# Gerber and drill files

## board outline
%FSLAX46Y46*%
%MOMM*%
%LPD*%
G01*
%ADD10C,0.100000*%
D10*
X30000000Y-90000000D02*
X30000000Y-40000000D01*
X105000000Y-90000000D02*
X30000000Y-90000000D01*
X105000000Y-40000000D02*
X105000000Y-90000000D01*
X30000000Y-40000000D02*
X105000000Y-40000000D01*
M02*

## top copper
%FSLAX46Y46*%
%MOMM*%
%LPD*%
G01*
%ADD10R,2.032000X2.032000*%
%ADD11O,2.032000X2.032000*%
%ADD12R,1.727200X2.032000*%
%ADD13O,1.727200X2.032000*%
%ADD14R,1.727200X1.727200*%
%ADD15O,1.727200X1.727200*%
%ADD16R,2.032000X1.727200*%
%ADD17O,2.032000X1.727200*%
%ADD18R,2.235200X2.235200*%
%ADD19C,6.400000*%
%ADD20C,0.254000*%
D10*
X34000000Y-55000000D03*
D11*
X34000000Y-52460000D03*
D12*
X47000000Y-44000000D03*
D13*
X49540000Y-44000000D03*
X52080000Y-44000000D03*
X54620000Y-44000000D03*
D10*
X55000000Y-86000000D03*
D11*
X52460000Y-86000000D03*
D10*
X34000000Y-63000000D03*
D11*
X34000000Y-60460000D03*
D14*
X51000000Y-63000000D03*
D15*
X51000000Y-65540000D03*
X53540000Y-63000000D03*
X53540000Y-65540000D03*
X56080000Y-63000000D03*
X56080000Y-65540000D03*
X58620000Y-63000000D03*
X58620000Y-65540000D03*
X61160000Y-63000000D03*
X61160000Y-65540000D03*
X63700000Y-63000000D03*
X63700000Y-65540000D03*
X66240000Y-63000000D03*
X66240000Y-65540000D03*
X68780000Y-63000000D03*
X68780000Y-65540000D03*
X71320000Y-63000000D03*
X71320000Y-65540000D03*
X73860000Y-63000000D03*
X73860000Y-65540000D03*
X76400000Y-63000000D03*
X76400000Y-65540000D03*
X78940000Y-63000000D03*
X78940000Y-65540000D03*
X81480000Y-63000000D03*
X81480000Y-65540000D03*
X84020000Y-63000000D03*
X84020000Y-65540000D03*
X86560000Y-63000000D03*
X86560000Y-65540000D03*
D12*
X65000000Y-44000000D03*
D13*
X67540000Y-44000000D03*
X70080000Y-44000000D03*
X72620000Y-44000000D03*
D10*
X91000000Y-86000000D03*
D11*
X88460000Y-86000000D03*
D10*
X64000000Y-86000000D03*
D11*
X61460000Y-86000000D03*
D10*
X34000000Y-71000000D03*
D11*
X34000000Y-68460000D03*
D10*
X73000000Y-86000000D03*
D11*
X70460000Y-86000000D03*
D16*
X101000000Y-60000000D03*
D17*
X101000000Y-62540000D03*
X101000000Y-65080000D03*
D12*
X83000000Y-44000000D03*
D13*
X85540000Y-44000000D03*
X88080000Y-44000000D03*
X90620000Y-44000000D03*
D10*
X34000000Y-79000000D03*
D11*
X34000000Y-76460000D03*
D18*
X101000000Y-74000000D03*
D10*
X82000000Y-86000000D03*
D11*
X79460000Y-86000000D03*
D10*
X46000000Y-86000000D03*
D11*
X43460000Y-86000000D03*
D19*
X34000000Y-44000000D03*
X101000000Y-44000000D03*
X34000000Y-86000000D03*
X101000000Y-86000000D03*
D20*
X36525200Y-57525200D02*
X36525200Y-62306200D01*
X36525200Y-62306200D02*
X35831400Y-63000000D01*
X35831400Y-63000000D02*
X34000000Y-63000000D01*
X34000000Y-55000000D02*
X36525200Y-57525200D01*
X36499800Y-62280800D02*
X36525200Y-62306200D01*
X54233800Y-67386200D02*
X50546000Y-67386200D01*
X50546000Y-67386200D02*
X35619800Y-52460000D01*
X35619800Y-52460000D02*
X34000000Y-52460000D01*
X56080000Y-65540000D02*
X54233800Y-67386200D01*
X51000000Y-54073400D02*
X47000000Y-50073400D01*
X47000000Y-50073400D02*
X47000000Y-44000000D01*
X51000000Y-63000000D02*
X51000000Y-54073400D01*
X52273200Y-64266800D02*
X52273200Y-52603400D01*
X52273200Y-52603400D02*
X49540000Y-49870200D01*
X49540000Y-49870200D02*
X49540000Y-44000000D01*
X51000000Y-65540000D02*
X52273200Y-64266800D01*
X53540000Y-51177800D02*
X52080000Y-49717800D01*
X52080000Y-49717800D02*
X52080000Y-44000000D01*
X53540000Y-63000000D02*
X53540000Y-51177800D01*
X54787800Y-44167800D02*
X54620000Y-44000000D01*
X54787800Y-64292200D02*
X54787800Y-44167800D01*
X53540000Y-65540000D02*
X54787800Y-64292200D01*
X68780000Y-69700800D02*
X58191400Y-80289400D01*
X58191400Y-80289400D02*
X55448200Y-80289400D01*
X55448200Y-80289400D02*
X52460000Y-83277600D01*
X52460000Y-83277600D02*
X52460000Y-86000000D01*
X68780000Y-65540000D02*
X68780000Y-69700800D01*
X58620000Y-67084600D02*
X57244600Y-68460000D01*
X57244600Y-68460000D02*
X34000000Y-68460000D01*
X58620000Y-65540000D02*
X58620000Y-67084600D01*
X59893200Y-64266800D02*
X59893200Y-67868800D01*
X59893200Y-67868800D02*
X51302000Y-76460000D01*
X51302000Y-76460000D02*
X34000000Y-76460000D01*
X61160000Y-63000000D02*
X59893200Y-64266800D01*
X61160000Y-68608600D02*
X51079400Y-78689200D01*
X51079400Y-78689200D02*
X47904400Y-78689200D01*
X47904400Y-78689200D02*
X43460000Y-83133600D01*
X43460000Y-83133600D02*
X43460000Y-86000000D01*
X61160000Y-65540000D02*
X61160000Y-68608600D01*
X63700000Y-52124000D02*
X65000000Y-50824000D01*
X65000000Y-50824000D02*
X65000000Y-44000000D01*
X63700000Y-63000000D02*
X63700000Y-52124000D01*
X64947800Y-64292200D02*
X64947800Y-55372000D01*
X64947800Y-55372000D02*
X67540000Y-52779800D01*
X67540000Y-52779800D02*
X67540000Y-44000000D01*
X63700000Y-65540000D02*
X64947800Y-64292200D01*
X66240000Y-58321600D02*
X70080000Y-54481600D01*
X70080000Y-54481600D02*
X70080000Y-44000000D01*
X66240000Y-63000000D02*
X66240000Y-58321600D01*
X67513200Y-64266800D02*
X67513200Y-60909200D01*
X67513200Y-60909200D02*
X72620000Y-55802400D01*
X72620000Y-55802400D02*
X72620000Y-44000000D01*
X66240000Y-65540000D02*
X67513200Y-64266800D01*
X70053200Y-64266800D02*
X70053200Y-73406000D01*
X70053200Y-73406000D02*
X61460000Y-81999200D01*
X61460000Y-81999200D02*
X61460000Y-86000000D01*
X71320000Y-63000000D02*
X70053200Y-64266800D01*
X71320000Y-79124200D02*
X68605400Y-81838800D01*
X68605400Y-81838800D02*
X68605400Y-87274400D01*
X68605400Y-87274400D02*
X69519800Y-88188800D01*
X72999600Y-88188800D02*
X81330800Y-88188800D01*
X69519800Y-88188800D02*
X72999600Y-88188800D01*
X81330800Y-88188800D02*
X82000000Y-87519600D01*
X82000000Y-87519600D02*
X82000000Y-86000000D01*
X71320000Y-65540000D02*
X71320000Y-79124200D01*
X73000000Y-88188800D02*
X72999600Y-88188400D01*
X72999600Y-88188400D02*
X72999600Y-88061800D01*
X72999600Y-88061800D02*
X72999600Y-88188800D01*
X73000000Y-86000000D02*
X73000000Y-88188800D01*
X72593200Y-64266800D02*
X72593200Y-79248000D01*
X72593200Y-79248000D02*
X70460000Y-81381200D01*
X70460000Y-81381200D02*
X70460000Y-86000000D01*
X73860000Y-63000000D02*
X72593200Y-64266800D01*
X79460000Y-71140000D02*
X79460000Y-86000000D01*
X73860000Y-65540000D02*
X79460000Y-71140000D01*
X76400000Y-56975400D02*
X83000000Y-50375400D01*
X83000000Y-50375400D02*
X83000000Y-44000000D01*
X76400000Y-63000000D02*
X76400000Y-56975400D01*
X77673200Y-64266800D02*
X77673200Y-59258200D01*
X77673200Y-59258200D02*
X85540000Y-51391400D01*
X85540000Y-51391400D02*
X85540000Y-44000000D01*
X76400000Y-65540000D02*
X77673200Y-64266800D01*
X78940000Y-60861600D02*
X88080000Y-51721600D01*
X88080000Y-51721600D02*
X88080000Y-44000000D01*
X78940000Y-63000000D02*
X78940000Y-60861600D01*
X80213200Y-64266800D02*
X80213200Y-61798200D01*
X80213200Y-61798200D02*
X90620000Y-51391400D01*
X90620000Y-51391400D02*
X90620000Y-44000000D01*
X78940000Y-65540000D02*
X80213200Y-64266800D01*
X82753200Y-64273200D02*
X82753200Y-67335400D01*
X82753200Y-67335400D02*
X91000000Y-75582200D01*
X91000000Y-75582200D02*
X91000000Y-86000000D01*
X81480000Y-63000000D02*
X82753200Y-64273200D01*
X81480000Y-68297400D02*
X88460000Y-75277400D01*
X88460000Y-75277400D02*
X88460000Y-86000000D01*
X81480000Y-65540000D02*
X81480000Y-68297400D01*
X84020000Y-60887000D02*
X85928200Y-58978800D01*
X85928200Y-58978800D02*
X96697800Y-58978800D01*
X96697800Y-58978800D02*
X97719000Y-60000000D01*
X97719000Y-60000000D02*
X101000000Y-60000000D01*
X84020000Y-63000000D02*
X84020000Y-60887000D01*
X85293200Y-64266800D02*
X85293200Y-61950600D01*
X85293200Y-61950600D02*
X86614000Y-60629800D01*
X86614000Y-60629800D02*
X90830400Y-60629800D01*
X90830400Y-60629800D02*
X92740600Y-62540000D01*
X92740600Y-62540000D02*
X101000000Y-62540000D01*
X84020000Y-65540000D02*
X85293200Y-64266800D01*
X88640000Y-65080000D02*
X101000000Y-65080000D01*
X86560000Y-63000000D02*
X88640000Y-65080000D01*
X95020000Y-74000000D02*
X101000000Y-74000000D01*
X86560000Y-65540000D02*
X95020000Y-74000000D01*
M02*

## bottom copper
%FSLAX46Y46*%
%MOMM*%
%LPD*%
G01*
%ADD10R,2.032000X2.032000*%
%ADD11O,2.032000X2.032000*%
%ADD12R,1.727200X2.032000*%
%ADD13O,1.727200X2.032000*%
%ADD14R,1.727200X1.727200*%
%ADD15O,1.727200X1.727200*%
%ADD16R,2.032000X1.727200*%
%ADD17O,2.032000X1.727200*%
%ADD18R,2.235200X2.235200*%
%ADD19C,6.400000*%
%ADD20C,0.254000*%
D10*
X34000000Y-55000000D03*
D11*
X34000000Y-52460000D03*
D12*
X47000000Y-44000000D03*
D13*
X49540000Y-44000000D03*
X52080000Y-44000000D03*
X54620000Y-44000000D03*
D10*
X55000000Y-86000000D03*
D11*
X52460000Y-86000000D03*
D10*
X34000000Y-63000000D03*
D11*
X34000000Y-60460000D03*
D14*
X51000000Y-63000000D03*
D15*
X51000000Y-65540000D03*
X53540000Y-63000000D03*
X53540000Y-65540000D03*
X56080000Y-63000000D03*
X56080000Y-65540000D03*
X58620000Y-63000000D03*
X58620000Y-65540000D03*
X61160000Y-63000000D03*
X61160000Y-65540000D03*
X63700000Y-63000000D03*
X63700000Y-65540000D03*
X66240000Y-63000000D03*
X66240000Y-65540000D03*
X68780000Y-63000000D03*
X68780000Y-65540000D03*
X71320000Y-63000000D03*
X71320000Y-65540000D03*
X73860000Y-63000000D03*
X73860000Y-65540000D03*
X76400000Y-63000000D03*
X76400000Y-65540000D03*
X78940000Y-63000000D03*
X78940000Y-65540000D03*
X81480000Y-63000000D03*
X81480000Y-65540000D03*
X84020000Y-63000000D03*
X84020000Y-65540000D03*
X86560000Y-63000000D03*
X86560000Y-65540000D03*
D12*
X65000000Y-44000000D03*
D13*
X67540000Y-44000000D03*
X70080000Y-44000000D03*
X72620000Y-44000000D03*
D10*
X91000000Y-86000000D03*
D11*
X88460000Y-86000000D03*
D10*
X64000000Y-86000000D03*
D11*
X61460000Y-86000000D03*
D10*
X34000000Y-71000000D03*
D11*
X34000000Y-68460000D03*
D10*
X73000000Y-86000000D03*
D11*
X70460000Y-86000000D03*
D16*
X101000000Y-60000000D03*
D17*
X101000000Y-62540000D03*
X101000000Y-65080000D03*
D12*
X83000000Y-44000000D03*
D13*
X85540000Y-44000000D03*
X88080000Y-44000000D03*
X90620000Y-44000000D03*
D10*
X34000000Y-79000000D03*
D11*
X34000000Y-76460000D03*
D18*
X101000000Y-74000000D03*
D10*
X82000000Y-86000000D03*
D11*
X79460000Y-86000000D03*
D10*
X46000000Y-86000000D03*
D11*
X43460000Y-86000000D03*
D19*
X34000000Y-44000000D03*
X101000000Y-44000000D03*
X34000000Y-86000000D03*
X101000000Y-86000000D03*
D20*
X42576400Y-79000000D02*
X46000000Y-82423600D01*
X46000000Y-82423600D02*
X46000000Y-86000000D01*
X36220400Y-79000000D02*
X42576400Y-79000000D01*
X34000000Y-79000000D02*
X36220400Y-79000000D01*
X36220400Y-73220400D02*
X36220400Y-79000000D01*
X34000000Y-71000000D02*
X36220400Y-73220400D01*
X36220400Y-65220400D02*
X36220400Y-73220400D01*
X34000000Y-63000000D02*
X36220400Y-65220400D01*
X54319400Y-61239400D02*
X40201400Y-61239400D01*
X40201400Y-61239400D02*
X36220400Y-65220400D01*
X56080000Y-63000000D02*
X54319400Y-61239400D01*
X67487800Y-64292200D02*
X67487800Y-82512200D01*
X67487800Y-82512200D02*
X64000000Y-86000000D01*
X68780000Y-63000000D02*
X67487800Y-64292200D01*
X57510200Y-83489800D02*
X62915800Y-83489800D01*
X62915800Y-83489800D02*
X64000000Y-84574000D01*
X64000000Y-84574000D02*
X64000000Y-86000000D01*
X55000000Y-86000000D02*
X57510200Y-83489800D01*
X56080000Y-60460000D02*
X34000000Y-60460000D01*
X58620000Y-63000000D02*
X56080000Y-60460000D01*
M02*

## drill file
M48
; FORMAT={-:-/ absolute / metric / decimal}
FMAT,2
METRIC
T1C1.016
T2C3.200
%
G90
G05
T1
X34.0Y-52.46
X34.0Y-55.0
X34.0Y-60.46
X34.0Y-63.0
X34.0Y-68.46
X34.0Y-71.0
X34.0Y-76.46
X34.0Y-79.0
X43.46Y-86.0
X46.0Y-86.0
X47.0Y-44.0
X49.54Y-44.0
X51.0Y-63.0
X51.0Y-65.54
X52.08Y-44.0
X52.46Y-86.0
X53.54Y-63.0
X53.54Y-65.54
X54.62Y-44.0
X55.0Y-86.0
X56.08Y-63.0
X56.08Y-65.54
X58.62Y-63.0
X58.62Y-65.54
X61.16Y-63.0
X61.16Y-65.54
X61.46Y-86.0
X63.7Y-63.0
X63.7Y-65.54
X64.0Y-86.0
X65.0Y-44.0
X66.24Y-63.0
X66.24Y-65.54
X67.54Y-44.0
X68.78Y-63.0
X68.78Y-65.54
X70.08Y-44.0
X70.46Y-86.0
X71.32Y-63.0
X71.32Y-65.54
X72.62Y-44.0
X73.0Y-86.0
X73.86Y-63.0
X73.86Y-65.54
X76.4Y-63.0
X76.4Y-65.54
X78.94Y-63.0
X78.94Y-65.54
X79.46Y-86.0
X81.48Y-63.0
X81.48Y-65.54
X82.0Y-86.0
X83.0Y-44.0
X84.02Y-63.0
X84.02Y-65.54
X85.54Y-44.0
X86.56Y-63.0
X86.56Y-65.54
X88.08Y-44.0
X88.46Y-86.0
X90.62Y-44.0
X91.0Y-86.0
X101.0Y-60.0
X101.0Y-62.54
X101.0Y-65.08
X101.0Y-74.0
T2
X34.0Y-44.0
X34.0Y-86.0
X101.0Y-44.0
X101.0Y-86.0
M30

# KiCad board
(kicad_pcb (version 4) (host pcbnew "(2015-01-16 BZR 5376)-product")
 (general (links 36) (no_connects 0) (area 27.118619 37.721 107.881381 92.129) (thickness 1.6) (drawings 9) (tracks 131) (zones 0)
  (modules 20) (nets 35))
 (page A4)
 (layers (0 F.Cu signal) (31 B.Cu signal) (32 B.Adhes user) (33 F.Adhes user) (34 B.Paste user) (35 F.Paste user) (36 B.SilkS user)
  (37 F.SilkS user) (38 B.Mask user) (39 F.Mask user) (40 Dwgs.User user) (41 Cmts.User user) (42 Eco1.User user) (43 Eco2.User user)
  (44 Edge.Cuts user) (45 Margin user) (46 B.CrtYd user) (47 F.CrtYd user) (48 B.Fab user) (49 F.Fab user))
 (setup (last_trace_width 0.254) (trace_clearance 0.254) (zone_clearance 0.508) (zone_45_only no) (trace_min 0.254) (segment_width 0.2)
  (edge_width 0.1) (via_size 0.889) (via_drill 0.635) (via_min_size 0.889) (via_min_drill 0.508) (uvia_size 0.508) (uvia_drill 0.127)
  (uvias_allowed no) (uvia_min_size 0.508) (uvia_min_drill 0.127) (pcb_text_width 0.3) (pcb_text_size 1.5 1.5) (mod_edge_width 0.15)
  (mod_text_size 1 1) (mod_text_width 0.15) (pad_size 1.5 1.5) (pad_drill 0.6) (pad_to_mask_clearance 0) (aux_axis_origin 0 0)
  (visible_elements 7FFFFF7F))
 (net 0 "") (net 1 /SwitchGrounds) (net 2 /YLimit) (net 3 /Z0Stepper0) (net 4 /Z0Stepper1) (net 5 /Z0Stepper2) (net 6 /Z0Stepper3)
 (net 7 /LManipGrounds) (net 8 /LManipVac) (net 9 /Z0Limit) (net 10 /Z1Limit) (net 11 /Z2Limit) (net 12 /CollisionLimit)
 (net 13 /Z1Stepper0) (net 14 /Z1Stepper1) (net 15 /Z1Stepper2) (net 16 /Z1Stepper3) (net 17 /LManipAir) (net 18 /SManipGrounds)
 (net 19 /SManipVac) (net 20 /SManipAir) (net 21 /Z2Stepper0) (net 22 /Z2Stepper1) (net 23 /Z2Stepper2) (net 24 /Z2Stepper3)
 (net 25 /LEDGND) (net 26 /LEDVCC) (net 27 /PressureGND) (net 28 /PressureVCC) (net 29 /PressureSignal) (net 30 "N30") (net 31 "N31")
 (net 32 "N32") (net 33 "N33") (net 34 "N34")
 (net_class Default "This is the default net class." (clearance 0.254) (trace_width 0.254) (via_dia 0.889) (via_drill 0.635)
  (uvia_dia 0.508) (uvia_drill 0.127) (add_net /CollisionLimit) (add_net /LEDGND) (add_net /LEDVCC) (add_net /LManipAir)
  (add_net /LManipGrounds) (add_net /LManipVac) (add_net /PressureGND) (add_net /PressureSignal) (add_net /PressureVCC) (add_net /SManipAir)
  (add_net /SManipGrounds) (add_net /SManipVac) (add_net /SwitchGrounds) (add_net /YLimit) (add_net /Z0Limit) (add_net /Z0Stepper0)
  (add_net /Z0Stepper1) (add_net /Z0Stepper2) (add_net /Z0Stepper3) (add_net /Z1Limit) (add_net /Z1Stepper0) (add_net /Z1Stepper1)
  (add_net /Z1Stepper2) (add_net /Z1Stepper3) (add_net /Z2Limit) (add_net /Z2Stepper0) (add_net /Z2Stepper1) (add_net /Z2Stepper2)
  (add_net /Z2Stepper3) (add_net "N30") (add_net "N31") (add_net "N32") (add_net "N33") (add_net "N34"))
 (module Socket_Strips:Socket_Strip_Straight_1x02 (layer F.Cu) (at 34 55 90)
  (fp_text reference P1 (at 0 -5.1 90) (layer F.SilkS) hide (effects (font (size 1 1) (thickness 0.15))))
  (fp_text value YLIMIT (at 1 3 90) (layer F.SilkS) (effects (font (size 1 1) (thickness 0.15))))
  (pad 1 thru_hole rect (at 0 0 90) (size 2.032 2.032) (drill 1.016) (layers *.Cu *.Mask) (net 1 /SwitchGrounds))
  (pad 2 thru_hole oval (at 2.54 0 90) (size 2.032 2.032) (drill 1.016) (layers *.Cu *.Mask) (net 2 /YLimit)))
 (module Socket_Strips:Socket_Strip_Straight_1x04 (layer F.Cu) (at 47 44)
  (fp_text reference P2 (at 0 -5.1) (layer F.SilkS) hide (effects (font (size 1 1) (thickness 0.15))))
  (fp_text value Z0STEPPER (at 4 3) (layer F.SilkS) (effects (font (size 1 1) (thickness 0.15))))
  (pad 1 thru_hole rect (at 0 0) (size 1.7272 2.032) (drill 1.016) (layers *.Cu *.Mask) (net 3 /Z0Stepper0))
  (pad 2 thru_hole oval (at 2.54 0) (size 1.7272 2.032) (drill 1.016) (layers *.Cu *.Mask) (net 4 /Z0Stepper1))
  (pad 3 thru_hole oval (at 5.08 0) (size 1.7272 2.032) (drill 1.016) (layers *.Cu *.Mask) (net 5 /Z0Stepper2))
  (pad 4 thru_hole oval (at 7.62 0) (size 1.7272 2.032) (drill 1.016) (layers *.Cu *.Mask) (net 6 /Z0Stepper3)))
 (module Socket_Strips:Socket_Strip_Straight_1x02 (layer F.Cu) (at 55 86 180)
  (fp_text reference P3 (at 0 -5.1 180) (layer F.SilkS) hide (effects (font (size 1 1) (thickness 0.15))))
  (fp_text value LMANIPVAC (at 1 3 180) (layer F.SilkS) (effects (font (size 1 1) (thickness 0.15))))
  (pad 1 thru_hole rect (at 0 0 180) (size 2.032 2.032) (drill 1.016) (layers *.Cu *.Mask) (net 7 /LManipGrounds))
  (pad 2 thru_hole oval (at 2.54 0 180) (size 2.032 2.032) (drill 1.016) (layers *.Cu *.Mask) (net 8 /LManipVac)))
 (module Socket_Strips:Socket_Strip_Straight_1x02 (layer F.Cu) (at 34 63 90)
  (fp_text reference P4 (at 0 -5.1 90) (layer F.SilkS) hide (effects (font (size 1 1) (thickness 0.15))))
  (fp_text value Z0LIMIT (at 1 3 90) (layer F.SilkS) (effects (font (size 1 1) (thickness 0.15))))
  (pad 1 thru_hole rect (at 0 0 90) (size 2.032 2.032) (drill 1.016) (layers *.Cu *.Mask) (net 1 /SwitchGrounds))
  (pad 2 thru_hole oval (at 2.54 0 90) (size 2.032 2.032) (drill 1.016) (layers *.Cu *.Mask) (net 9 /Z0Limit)))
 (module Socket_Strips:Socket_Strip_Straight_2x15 (layer F.Cu) (at 51 63)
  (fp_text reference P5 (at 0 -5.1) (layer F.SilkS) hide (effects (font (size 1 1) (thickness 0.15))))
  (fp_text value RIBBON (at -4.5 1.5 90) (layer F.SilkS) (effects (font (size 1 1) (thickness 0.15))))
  (pad 1 thru_hole rect (at 0 0) (size 1.7272 1.7272) (drill 1.016) (layers *.Cu *.Mask) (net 3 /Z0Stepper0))
  (pad 2 thru_hole oval (at 0 2.54) (size 1.7272 1.7272) (drill 1.016) (layers *.Cu *.Mask) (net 4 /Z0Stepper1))
  (pad 3 thru_hole oval (at 2.54 0) (size 1.7272 1.7272) (drill 1.016) (layers *.Cu *.Mask) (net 5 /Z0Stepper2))
  (pad 4 thru_hole oval (at 2.54 2.54) (size 1.7272 1.7272) (drill 1.016) (layers *.Cu *.Mask) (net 6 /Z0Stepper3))
  (pad 5 thru_hole oval (at 5.08 0) (size 1.7272 1.7272) (drill 1.016) (layers *.Cu *.Mask) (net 1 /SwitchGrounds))
  (pad 6 thru_hole oval (at 5.08 2.54) (size 1.7272 1.7272) (drill 1.016) (layers *.Cu *.Mask) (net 2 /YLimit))
  (pad 7 thru_hole oval (at 7.62 0) (size 1.7272 1.7272) (drill 1.016) (layers *.Cu *.Mask) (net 9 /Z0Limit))
  (pad 8 thru_hole oval (at 7.62 2.54) (size 1.7272 1.7272) (drill 1.016) (layers *.Cu *.Mask) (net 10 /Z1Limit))
  (pad 9 thru_hole oval (at 10.16 0) (size 1.7272 1.7272) (drill 1.016) (layers *.Cu *.Mask) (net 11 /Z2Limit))
  (pad 10 thru_hole oval (at 10.16 2.54) (size 1.7272 1.7272) (drill 1.016) (layers *.Cu *.Mask) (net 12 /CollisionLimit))
  (pad 11 thru_hole oval (at 12.7 0) (size 1.7272 1.7272) (drill 1.016) (layers *.Cu *.Mask) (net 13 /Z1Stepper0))
  (pad 12 thru_hole oval (at 12.7 2.54) (size 1.7272 1.7272) (drill 1.016) (layers *.Cu *.Mask) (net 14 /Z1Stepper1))
  (pad 13 thru_hole oval (at 15.24 0) (size 1.7272 1.7272) (drill 1.016) (layers *.Cu *.Mask) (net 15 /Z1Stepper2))
  (pad 14 thru_hole oval (at 15.24 2.54) (size 1.7272 1.7272) (drill 1.016) (layers *.Cu *.Mask) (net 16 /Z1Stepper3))
  (pad 15 thru_hole oval (at 17.78 0) (size 1.7272 1.7272) (drill 1.016) (layers *.Cu *.Mask) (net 7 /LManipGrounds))
  (pad 16 thru_hole oval (at 17.78 2.54) (size 1.7272 1.7272) (drill 1.016) (layers *.Cu *.Mask) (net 8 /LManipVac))
  (pad 17 thru_hole oval (at 20.32 0) (size 1.7272 1.7272) (drill 1.016) (layers *.Cu *.Mask) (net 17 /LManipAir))
  (pad 18 thru_hole oval (at 20.32 2.54) (size 1.7272 1.7272) (drill 1.016) (layers *.Cu *.Mask) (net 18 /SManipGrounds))
  (pad 19 thru_hole oval (at 22.86 0) (size 1.7272 1.7272) (drill 1.016) (layers *.Cu *.Mask) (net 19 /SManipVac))
  (pad 20 thru_hole oval (at 22.86 2.54) (size 1.7272 1.7272) (drill 1.016) (layers *.Cu *.Mask) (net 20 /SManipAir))
  (pad 21 thru_hole oval (at 25.4 0) (size 1.7272 1.7272) (drill 1.016) (layers *.Cu *.Mask) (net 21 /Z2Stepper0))
  (pad 22 thru_hole oval (at 25.4 2.54) (size 1.7272 1.7272) (drill 1.016) (layers *.Cu *.Mask) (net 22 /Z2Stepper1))
  (pad 23 thru_hole oval (at 27.94 0) (size 1.7272 1.7272) (drill 1.016) (layers *.Cu *.Mask) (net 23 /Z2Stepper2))
  (pad 24 thru_hole oval (at 27.94 2.54) (size 1.7272 1.7272) (drill 1.016) (layers *.Cu *.Mask) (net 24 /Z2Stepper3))
  (pad 25 thru_hole oval (at 30.48 0) (size 1.7272 1.7272) (drill 1.016) (layers *.Cu *.Mask) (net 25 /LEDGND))
  (pad 26 thru_hole oval (at 30.48 2.54) (size 1.7272 1.7272) (drill 1.016) (layers *.Cu *.Mask) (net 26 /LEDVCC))
  (pad 27 thru_hole oval (at 33.02 0) (size 1.7272 1.7272) (drill 1.016) (layers *.Cu *.Mask) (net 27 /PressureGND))
  (pad 28 thru_hole oval (at 33.02 2.54) (size 1.7272 1.7272) (drill 1.016) (layers *.Cu *.Mask) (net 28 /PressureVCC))
  (pad 29 thru_hole oval (at 35.56 0) (size 1.7272 1.7272) (drill 1.016) (layers *.Cu *.Mask) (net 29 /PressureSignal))
  (pad 30 thru_hole oval (at 35.56 2.54) (size 1.7272 1.7272) (drill 1.016) (layers *.Cu *.Mask) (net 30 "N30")))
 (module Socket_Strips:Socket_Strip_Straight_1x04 (layer F.Cu) (at 65 44)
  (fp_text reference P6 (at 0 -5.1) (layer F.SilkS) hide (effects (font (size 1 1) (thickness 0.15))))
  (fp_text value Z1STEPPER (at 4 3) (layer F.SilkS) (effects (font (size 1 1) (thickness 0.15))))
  (pad 1 thru_hole rect (at 0 0) (size 1.7272 2.032) (drill 1.016) (layers *.Cu *.Mask) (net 13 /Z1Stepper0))
  (pad 2 thru_hole oval (at 2.54 0) (size 1.7272 2.032) (drill 1.016) (layers *.Cu *.Mask) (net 14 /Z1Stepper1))
  (pad 3 thru_hole oval (at 5.08 0) (size 1.7272 2.032) (drill 1.016) (layers *.Cu *.Mask) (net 15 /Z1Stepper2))
  (pad 4 thru_hole oval (at 7.62 0) (size 1.7272 2.032) (drill 1.016) (layers *.Cu *.Mask) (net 16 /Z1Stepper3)))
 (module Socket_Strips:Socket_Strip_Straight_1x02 (layer F.Cu) (at 91 86 180)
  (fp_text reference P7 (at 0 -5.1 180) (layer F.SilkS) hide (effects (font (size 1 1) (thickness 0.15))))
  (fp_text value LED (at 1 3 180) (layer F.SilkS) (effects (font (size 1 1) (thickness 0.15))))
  (pad 1 thru_hole rect (at 0 0 180) (size 2.032 2.032) (drill 1.016) (layers *.Cu *.Mask) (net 25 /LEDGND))
  (pad 2 thru_hole oval (at 2.54 0 180) (size 2.032 2.032) (drill 1.016) (layers *.Cu *.Mask) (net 26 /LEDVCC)))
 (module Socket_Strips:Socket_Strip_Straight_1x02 (layer F.Cu) (at 64 86 180)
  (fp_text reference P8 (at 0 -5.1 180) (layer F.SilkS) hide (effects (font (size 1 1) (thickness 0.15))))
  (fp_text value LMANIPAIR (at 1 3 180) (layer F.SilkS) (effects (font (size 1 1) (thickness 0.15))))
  (pad 1 thru_hole rect (at 0 0 180) (size 2.032 2.032) (drill 1.016) (layers *.Cu *.Mask) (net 7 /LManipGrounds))
  (pad 2 thru_hole oval (at 2.54 0 180) (size 2.032 2.032) (drill 1.016) (layers *.Cu *.Mask) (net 17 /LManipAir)))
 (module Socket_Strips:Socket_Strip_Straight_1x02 (layer F.Cu) (at 34 71 90)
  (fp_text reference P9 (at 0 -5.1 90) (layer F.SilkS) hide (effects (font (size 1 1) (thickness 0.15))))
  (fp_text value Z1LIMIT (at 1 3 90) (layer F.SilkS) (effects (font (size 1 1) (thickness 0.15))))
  (pad 1 thru_hole rect (at 0 0 90) (size 2.032 2.032) (drill 1.016) (layers *.Cu *.Mask) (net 1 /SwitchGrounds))
  (pad 2 thru_hole oval (at 2.54 0 90) (size 2.032 2.032) (drill 1.016) (layers *.Cu *.Mask) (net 10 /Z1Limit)))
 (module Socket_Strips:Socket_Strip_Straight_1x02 (layer F.Cu) (at 73 86 180)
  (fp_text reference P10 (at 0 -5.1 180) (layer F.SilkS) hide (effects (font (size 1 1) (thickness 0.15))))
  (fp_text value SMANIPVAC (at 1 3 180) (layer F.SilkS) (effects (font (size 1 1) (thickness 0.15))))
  (pad 1 thru_hole rect (at 0 0 180) (size 2.032 2.032) (drill 1.016) (layers *.Cu *.Mask) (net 18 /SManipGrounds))
  (pad 2 thru_hole oval (at 2.54 0 180) (size 2.032 2.032) (drill 1.016) (layers *.Cu *.Mask) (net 19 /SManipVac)))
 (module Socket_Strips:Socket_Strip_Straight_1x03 (layer F.Cu) (at 101 60 270)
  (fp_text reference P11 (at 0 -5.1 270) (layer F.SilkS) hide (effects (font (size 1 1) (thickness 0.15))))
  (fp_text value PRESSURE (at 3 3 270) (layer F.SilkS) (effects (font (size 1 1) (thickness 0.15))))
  (pad 1 thru_hole rect (at 0 0 270) (size 1.7272 2.032) (drill 1.016) (layers *.Cu *.Mask) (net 27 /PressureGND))
  (pad 2 thru_hole oval (at 2.54 0 270) (size 1.7272 2.032) (drill 1.016) (layers *.Cu *.Mask) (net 28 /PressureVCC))
  (pad 3 thru_hole oval (at 5.08 0 270) (size 1.7272 2.032) (drill 1.016) (layers *.Cu *.Mask) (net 29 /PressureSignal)))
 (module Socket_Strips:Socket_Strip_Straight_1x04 (layer F.Cu) (at 83 44)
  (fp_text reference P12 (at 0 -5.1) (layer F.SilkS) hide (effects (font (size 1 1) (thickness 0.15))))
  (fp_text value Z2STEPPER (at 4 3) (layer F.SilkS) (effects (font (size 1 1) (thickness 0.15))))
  (pad 1 thru_hole rect (at 0 0) (size 1.7272 2.032) (drill 1.016) (layers *.Cu *.Mask) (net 21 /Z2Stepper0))
  (pad 2 thru_hole oval (at 2.54 0) (size 1.7272 2.032) (drill 1.016) (layers *.Cu *.Mask) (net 22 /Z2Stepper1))
  (pad 3 thru_hole oval (at 5.08 0) (size 1.7272 2.032) (drill 1.016) (layers *.Cu *.Mask) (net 23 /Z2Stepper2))
  (pad 4 thru_hole oval (at 7.62 0) (size 1.7272 2.032) (drill 1.016) (layers *.Cu *.Mask) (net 24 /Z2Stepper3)))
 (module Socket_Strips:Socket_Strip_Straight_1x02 (layer F.Cu) (at 34 79 90)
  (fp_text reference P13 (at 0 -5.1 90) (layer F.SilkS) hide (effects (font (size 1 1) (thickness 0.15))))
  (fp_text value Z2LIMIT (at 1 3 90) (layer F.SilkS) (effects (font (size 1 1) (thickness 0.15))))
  (pad 1 thru_hole rect (at 0 0 90) (size 2.032 2.032) (drill 1.016) (layers *.Cu *.Mask) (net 1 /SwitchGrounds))
  (pad 2 thru_hole oval (at 2.54 0 90) (size 2.032 2.032) (drill 1.016) (layers *.Cu *.Mask) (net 11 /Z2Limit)))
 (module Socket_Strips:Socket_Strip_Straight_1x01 (layer F.Cu) (at 101 74)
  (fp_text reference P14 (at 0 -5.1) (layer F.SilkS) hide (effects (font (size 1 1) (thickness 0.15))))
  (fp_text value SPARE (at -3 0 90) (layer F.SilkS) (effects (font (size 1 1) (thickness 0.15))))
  (pad 1 thru_hole rect (at 0 0) (size 2.2352 2.2352) (drill 1.016) (layers *.Cu *.Mask) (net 30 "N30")))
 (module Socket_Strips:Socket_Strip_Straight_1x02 (layer F.Cu) (at 82 86 180)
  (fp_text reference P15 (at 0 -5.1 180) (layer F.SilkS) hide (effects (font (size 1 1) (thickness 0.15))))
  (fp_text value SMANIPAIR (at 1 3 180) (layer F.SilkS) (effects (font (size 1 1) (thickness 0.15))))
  (pad 1 thru_hole rect (at 0 0 180) (size 2.032 2.032) (drill 1.016) (layers *.Cu *.Mask) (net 18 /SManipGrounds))
  (pad 2 thru_hole oval (at 2.54 0 180) (size 2.032 2.032) (drill 1.016) (layers *.Cu *.Mask) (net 20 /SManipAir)))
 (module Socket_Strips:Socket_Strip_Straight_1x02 (layer F.Cu) (at 46 86 180)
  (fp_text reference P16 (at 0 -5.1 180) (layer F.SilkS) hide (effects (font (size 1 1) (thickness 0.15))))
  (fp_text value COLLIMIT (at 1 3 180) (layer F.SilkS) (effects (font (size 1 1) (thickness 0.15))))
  (pad 1 thru_hole rect (at 0 0 180) (size 2.032 2.032) (drill 1.016) (layers *.Cu *.Mask) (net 1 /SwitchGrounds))
  (pad 2 thru_hole oval (at 2.54 0 180) (size 2.032 2.032) (drill 1.016) (layers *.Cu *.Mask) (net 12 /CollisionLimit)))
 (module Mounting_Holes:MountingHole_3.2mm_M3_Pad (layer F.Cu) (at 34 44)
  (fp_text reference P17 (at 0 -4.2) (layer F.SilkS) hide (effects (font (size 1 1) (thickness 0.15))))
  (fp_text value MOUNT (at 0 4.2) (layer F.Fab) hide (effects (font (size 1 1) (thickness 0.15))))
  (pad 1 thru_hole circle (at 0 0) (size 6.4 6.4) (drill 3.2) (layers *.Cu *.Mask) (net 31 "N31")))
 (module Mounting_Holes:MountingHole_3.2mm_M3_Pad (layer F.Cu) (at 101 44)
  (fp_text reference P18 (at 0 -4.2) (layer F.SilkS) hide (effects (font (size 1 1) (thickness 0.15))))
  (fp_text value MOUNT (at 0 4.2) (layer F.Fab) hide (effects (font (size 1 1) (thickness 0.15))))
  (pad 1 thru_hole circle (at 0 0) (size 6.4 6.4) (drill 3.2) (layers *.Cu *.Mask) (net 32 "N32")))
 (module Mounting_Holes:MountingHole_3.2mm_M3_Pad (layer F.Cu) (at 34 86)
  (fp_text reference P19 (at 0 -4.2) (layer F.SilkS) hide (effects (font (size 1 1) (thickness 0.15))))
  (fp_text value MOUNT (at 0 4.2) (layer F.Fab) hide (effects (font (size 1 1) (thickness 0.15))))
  (pad 1 thru_hole circle (at 0 0) (size 6.4 6.4) (drill 3.2) (layers *.Cu *.Mask) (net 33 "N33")))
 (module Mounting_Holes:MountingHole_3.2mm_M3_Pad (layer F.Cu) (at 101 86)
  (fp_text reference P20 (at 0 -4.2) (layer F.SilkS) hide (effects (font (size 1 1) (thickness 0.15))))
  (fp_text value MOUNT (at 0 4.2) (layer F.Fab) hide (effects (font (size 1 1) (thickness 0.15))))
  (pad 1 thru_hole circle (at 0 0) (size 6.4 6.4) (drill 3.2) (layers *.Cu *.Mask) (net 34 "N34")))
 (gr_line (start 30 90) (end 30 40) (angle 90) (layer Edge.Cuts) (width 0.1))
 (gr_line (start 105 90) (end 30 90) (angle 90) (layer Edge.Cuts) (width 0.1))
 (gr_line (start 105 40) (end 105 90) (angle 90) (layer Edge.Cuts) (width 0.1))
 (gr_line (start 30 40) (end 105 40) (angle 90) (layer Edge.Cuts) (width 0.1))
 (segment (start 42.5764 79) (end 46 82.4236) (width 0.254) (layer B.Cu) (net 1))
 (segment (start 46 82.4236) (end 46 86) (width 0.254) (layer B.Cu) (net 1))
 (segment (start 36.2204 79) (end 42.5764 79) (width 0.254) (layer B.Cu) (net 1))
 (segment (start 34 79) (end 36.2204 79) (width 0.254) (layer B.Cu) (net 1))
 (segment (start 36.2204 73.2204) (end 36.2204 79) (width 0.254) (layer B.Cu) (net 1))
 (segment (start 34 71) (end 36.2204 73.2204) (width 0.254) (layer B.Cu) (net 1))
 (segment (start 36.2204 65.2204) (end 36.2204 73.2204) (width 0.254) (layer B.Cu) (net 1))
 (segment (start 34 63) (end 36.2204 65.2204) (width 0.254) (layer B.Cu) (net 1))
 (segment (start 36.5252 57.5252) (end 36.5252 62.3062) (width 0.254) (layer F.Cu) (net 1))
 (segment (start 36.5252 62.3062) (end 35.8314 63) (width 0.254) (layer F.Cu) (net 1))
 (segment (start 35.8314 63) (end 34 63) (width 0.254) (layer F.Cu) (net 1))
 (segment (start 34 55) (end 36.5252 57.5252) (width 0.254) (layer F.Cu) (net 1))
 (segment (start 36.4998 62.2808) (end 36.5252 62.3062) (width 0.254) (layer F.Cu) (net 1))
 (segment (start 54.3194 61.2394) (end 40.2014 61.2394) (width 0.254) (layer B.Cu) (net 1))
 (segment (start 40.2014 61.2394) (end 36.2204 65.2204) (width 0.254) (layer B.Cu) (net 1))
 (segment (start 56.08 63) (end 54.3194 61.2394) (width 0.254) (layer B.Cu) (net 1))
 (segment (start 54.2338 67.3862) (end 50.546 67.3862) (width 0.254) (layer F.Cu) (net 2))
 (segment (start 50.546 67.3862) (end 35.6198 52.46) (width 0.254) (layer F.Cu) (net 2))
 (segment (start 35.6198 52.46) (end 34 52.46) (width 0.254) (layer F.Cu) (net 2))
 (segment (start 56.08 65.54) (end 54.2338 67.3862) (width 0.254) (layer F.Cu) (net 2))
 (segment (start 51 54.0734) (end 47 50.0734) (width 0.254) (layer F.Cu) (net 3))
 (segment (start 47 50.0734) (end 47 44) (width 0.254) (layer F.Cu) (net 3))
 (segment (start 51 63) (end 51 54.0734) (width 0.254) (layer F.Cu) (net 3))
 (segment (start 52.2732 64.2668) (end 52.2732 52.6034) (width 0.254) (layer F.Cu) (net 4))
 (segment (start 52.2732 52.6034) (end 49.54 49.8702) (width 0.254) (layer F.Cu) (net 4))
 (segment (start 49.54 49.8702) (end 49.54 44) (width 0.254) (layer F.Cu) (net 4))
 (segment (start 51 65.54) (end 52.2732 64.2668) (width 0.254) (layer F.Cu) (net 4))
 (segment (start 53.54 51.1778) (end 52.08 49.7178) (width 0.254) (layer F.Cu) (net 5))
 (segment (start 52.08 49.7178) (end 52.08 44) (width 0.254) (layer F.Cu) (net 5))
 (segment (start 53.54 63) (end 53.54 51.1778) (width 0.254) (layer F.Cu) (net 5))
 (segment (start 54.7878 44.1678) (end 54.62 44) (width 0.254) (layer F.Cu) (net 6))
 (segment (start 54.7878 64.2922) (end 54.7878 44.1678) (width 0.254) (layer F.Cu) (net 6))
 (segment (start 53.54 65.54) (end 54.7878 64.2922) (width 0.254) (layer F.Cu) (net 6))
 (segment (start 67.4878 64.2922) (end 67.4878 82.5122) (width 0.254) (layer B.Cu) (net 7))
 (segment (start 67.4878 82.5122) (end 64 86) (width 0.254) (layer B.Cu) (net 7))
 (segment (start 68.78 63) (end 67.4878 64.2922) (width 0.254) (layer B.Cu) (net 7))
 (segment (start 57.5102 83.4898) (end 62.9158 83.4898) (width 0.254) (layer B.Cu) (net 7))
 (segment (start 62.9158 83.4898) (end 64 84.574) (width 0.254) (layer B.Cu) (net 7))
 (segment (start 64 84.574) (end 64 86) (width 0.254) (layer B.Cu) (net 7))
 (segment (start 55 86) (end 57.5102 83.4898) (width 0.254) (layer B.Cu) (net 7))
 (segment (start 68.78 69.7008) (end 58.1914 80.2894) (width 0.254) (layer F.Cu) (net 8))
 (segment (start 58.1914 80.2894) (end 55.4482 80.2894) (width 0.254) (layer F.Cu) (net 8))
 (segment (start 55.4482 80.2894) (end 52.46 83.2776) (width 0.254) (layer F.Cu) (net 8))
 (segment (start 52.46 83.2776) (end 52.46 86) (width 0.254) (layer F.Cu) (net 8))
 (segment (start 68.78 65.54) (end 68.78 69.7008) (width 0.254) (layer F.Cu) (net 8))
 (segment (start 56.08 60.46) (end 34 60.46) (width 0.254) (layer B.Cu) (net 9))
 (segment (start 58.62 63) (end 56.08 60.46) (width 0.254) (layer B.Cu) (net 9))
 (segment (start 58.62 67.0846) (end 57.2446 68.46) (width 0.254) (layer F.Cu) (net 10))
 (segment (start 57.2446 68.46) (end 34 68.46) (width 0.254) (layer F.Cu) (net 10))
 (segment (start 58.62 65.54) (end 58.62 67.0846) (width 0.254) (layer F.Cu) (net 10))
 (segment (start 59.8932 64.2668) (end 59.8932 67.8688) (width 0.254) (layer F.Cu) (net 11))
 (segment (start 59.8932 67.8688) (end 51.302 76.46) (width 0.254) (layer F.Cu) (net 11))
 (segment (start 51.302 76.46) (end 34 76.46) (width 0.254) (layer F.Cu) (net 11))
 (segment (start 61.16 63) (end 59.8932 64.2668) (width 0.254) (layer F.Cu) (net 11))
 (segment (start 61.16 68.6086) (end 51.0794 78.6892) (width 0.254) (layer F.Cu) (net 12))
 (segment (start 51.0794 78.6892) (end 47.9044 78.6892) (width 0.254) (layer F.Cu) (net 12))
 (segment (start 47.9044 78.6892) (end 43.46 83.1336) (width 0.254) (layer F.Cu) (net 12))
 (segment (start 43.46 83.1336) (end 43.46 86) (width 0.254) (layer F.Cu) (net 12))
 (segment (start 61.16 65.54) (end 61.16 68.6086) (width 0.254) (layer F.Cu) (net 12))
 (segment (start 63.7 52.124) (end 65 50.824) (width 0.254) (layer F.Cu) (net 13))
 (segment (start 65 50.824) (end 65 44) (width 0.254) (layer F.Cu) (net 13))
 (segment (start 63.7 63) (end 63.7 52.124) (width 0.254) (layer F.Cu) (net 13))
 (segment (start 64.9478 64.2922) (end 64.9478 55.372) (width 0.254) (layer F.Cu) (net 14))
 (segment (start 64.9478 55.372) (end 67.54 52.7798) (width 0.254) (layer F.Cu) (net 14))
 (segment (start 67.54 52.7798) (end 67.54 44) (width 0.254) (layer F.Cu) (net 14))
 (segment (start 63.7 65.54) (end 64.9478 64.2922) (width 0.254) (layer F.Cu) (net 14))
 (segment (start 66.24 58.3216) (end 70.08 54.4816) (width 0.254) (layer F.Cu) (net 15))
 (segment (start 70.08 54.4816) (end 70.08 44) (width 0.254) (layer F.Cu) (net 15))
 (segment (start 66.24 63) (end 66.24 58.3216) (width 0.254) (layer F.Cu) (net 15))
 (segment (start 67.5132 64.2668) (end 67.5132 60.9092) (width 0.254) (layer F.Cu) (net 16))
 (segment (start 67.5132 60.9092) (end 72.62 55.8024) (width 0.254) (layer F.Cu) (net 16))
 (segment (start 72.62 55.8024) (end 72.62 44) (width 0.254) (layer F.Cu) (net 16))
 (segment (start 66.24 65.54) (end 67.5132 64.2668) (width 0.254) (layer F.Cu) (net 16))
 (segment (start 70.0532 64.2668) (end 70.0532 73.406) (width 0.254) (layer F.Cu) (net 17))
 (segment (start 70.0532 73.406) (end 61.46 81.9992) (width 0.254) (layer F.Cu) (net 17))
 (segment (start 61.46 81.9992) (end 61.46 86) (width 0.254) (layer F.Cu) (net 17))
 (segment (start 71.32 63) (end 70.0532 64.2668) (width 0.254) (layer F.Cu) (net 17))
 (segment (start 71.32 79.1242) (end 68.6054 81.8388) (width 0.254) (layer F.Cu) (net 18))
 (segment (start 68.6054 81.8388) (end 68.6054 87.2744) (width 0.254) (layer F.Cu) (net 18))
 (segment (start 68.6054 87.2744) (end 69.5198 88.1888) (width 0.254) (layer F.Cu) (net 18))
 (segment (start 72.9996 88.1888) (end 81.3308 88.1888) (width 0.254) (layer F.Cu) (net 18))
 (segment (start 69.5198 88.1888) (end 72.9996 88.1888) (width 0.254) (layer F.Cu) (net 18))
 (segment (start 81.3308 88.1888) (end 82 87.5196) (width 0.254) (layer F.Cu) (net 18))
 (segment (start 82 87.5196) (end 82 86) (width 0.254) (layer F.Cu) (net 18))
 (segment (start 71.32 65.54) (end 71.32 79.1242) (width 0.254) (layer F.Cu) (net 18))
 (segment (start 73 88.1888) (end 72.9996 88.1884) (width 0.254) (layer F.Cu) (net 18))
 (segment (start 72.9996 88.1884) (end 72.9996 88.0618) (width 0.254) (layer F.Cu) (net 18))
 (segment (start 72.9996 88.0618) (end 72.9996 88.1888) (width 0.254) (layer F.Cu) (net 18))
 (segment (start 73 86) (end 73 88.1888) (width 0.254) (layer F.Cu) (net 18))
 (segment (start 72.5932 64.2668) (end 72.5932 79.248) (width 0.254) (layer F.Cu) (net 19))
 (segment (start 72.5932 79.248) (end 70.46 81.3812) (width 0.254) (layer F.Cu) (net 19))
 (segment (start 70.46 81.3812) (end 70.46 86) (width 0.254) (layer F.Cu) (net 19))
 (segment (start 73.86 63) (end 72.5932 64.2668) (width 0.254) (layer F.Cu) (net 19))
 (segment (start 79.46 71.14) (end 79.46 86) (width 0.254) (layer F.Cu) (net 20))
 (segment (start 73.86 65.54) (end 79.46 71.14) (width 0.254) (layer F.Cu) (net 20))
 (segment (start 76.4 56.9754) (end 83 50.3754) (width 0.254) (layer F.Cu) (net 21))
 (segment (start 83 50.3754) (end 83 44) (width 0.254) (layer F.Cu) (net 21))
 (segment (start 76.4 63) (end 76.4 56.9754) (width 0.254) (layer F.Cu) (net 21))
 (segment (start 77.6732 64.2668) (end 77.6732 59.2582) (width 0.254) (layer F.Cu) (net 22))
 (segment (start 77.6732 59.2582) (end 85.54 51.3914) (width 0.254) (layer F.Cu) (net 22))
 (segment (start 85.54 51.3914) (end 85.54 44) (width 0.254) (layer F.Cu) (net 22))
 (segment (start 76.4 65.54) (end 77.6732 64.2668) (width 0.254) (layer F.Cu) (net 22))
 (segment (start 78.94 60.8616) (end 88.08 51.7216) (width 0.254) (layer F.Cu) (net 23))
 (segment (start 88.08 51.7216) (end 88.08 44) (width 0.254) (layer F.Cu) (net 23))
 (segment (start 78.94 63) (end 78.94 60.8616) (width 0.254) (layer F.Cu) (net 23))
 (segment (start 80.2132 64.2668) (end 80.2132 61.7982) (width 0.254) (layer F.Cu) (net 24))
 (segment (start 80.2132 61.7982) (end 90.62 51.3914) (width 0.254) (layer F.Cu) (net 24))
 (segment (start 90.62 51.3914) (end 90.62 44) (width 0.254) (layer F.Cu) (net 24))
 (segment (start 78.94 65.54) (end 80.2132 64.2668) (width 0.254) (layer F.Cu) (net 24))
 (segment (start 82.7532 64.2732) (end 82.7532 67.3354) (width 0.254) (layer F.Cu) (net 25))
 (segment (start 82.7532 67.3354) (end 91 75.5822) (width 0.254) (layer F.Cu) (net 25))
 (segment (start 91 75.5822) (end 91 86) (width 0.254) (layer F.Cu) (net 25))
 (segment (start 81.48 63) (end 82.7532 64.2732) (width 0.254) (layer F.Cu) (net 25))
 (segment (start 81.48 68.2974) (end 88.46 75.2774) (width 0.254) (layer F.Cu) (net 26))
 (segment (start 88.46 75.2774) (end 88.46 86) (width 0.254) (layer F.Cu) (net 26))
 (segment (start 81.48 65.54) (end 81.48 68.2974) (width 0.254) (layer F.Cu) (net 26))
 (segment (start 84.02 60.887) (end 85.9282 58.9788) (width 0.254) (layer F.Cu) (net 27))
 (segment (start 85.9282 58.9788) (end 96.6978 58.9788) (width 0.254) (layer F.Cu) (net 27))
 (segment (start 96.6978 58.9788) (end 97.719 60) (width 0.254) (layer F.Cu) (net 27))
 (segment (start 97.719 60) (end 101 60) (width 0.254) (layer F.Cu) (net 27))
 (segment (start 84.02 63) (end 84.02 60.887) (width 0.254) (layer F.Cu) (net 27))
 (segment (start 85.2932 64.2668) (end 85.2932 61.9506) (width 0.254) (layer F.Cu) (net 28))
 (segment (start 85.2932 61.9506) (end 86.614 60.6298) (width 0.254) (layer F.Cu) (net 28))
 (segment (start 86.614 60.6298) (end 90.8304 60.6298) (width 0.254) (layer F.Cu) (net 28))
 (segment (start 90.8304 60.6298) (end 92.7406 62.54) (width 0.254) (layer F.Cu) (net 28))
 (segment (start 92.7406 62.54) (end 101 62.54) (width 0.254) (layer F.Cu) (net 28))
 (segment (start 84.02 65.54) (end 85.2932 64.2668) (width 0.254) (layer F.Cu) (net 28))
 (segment (start 88.64 65.08) (end 101 65.08) (width 0.254) (layer F.Cu) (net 29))
 (segment (start 86.56 63) (end 88.64 65.08) (width 0.254) (layer F.Cu) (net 29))
 (segment (start 95.02 74) (end 101 74) (width 0.254) (layer F.Cu) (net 30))
 (segment (start 86.56 65.54) (end 95.02 74) (width 0.254) (layer F.Cu) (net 30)))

